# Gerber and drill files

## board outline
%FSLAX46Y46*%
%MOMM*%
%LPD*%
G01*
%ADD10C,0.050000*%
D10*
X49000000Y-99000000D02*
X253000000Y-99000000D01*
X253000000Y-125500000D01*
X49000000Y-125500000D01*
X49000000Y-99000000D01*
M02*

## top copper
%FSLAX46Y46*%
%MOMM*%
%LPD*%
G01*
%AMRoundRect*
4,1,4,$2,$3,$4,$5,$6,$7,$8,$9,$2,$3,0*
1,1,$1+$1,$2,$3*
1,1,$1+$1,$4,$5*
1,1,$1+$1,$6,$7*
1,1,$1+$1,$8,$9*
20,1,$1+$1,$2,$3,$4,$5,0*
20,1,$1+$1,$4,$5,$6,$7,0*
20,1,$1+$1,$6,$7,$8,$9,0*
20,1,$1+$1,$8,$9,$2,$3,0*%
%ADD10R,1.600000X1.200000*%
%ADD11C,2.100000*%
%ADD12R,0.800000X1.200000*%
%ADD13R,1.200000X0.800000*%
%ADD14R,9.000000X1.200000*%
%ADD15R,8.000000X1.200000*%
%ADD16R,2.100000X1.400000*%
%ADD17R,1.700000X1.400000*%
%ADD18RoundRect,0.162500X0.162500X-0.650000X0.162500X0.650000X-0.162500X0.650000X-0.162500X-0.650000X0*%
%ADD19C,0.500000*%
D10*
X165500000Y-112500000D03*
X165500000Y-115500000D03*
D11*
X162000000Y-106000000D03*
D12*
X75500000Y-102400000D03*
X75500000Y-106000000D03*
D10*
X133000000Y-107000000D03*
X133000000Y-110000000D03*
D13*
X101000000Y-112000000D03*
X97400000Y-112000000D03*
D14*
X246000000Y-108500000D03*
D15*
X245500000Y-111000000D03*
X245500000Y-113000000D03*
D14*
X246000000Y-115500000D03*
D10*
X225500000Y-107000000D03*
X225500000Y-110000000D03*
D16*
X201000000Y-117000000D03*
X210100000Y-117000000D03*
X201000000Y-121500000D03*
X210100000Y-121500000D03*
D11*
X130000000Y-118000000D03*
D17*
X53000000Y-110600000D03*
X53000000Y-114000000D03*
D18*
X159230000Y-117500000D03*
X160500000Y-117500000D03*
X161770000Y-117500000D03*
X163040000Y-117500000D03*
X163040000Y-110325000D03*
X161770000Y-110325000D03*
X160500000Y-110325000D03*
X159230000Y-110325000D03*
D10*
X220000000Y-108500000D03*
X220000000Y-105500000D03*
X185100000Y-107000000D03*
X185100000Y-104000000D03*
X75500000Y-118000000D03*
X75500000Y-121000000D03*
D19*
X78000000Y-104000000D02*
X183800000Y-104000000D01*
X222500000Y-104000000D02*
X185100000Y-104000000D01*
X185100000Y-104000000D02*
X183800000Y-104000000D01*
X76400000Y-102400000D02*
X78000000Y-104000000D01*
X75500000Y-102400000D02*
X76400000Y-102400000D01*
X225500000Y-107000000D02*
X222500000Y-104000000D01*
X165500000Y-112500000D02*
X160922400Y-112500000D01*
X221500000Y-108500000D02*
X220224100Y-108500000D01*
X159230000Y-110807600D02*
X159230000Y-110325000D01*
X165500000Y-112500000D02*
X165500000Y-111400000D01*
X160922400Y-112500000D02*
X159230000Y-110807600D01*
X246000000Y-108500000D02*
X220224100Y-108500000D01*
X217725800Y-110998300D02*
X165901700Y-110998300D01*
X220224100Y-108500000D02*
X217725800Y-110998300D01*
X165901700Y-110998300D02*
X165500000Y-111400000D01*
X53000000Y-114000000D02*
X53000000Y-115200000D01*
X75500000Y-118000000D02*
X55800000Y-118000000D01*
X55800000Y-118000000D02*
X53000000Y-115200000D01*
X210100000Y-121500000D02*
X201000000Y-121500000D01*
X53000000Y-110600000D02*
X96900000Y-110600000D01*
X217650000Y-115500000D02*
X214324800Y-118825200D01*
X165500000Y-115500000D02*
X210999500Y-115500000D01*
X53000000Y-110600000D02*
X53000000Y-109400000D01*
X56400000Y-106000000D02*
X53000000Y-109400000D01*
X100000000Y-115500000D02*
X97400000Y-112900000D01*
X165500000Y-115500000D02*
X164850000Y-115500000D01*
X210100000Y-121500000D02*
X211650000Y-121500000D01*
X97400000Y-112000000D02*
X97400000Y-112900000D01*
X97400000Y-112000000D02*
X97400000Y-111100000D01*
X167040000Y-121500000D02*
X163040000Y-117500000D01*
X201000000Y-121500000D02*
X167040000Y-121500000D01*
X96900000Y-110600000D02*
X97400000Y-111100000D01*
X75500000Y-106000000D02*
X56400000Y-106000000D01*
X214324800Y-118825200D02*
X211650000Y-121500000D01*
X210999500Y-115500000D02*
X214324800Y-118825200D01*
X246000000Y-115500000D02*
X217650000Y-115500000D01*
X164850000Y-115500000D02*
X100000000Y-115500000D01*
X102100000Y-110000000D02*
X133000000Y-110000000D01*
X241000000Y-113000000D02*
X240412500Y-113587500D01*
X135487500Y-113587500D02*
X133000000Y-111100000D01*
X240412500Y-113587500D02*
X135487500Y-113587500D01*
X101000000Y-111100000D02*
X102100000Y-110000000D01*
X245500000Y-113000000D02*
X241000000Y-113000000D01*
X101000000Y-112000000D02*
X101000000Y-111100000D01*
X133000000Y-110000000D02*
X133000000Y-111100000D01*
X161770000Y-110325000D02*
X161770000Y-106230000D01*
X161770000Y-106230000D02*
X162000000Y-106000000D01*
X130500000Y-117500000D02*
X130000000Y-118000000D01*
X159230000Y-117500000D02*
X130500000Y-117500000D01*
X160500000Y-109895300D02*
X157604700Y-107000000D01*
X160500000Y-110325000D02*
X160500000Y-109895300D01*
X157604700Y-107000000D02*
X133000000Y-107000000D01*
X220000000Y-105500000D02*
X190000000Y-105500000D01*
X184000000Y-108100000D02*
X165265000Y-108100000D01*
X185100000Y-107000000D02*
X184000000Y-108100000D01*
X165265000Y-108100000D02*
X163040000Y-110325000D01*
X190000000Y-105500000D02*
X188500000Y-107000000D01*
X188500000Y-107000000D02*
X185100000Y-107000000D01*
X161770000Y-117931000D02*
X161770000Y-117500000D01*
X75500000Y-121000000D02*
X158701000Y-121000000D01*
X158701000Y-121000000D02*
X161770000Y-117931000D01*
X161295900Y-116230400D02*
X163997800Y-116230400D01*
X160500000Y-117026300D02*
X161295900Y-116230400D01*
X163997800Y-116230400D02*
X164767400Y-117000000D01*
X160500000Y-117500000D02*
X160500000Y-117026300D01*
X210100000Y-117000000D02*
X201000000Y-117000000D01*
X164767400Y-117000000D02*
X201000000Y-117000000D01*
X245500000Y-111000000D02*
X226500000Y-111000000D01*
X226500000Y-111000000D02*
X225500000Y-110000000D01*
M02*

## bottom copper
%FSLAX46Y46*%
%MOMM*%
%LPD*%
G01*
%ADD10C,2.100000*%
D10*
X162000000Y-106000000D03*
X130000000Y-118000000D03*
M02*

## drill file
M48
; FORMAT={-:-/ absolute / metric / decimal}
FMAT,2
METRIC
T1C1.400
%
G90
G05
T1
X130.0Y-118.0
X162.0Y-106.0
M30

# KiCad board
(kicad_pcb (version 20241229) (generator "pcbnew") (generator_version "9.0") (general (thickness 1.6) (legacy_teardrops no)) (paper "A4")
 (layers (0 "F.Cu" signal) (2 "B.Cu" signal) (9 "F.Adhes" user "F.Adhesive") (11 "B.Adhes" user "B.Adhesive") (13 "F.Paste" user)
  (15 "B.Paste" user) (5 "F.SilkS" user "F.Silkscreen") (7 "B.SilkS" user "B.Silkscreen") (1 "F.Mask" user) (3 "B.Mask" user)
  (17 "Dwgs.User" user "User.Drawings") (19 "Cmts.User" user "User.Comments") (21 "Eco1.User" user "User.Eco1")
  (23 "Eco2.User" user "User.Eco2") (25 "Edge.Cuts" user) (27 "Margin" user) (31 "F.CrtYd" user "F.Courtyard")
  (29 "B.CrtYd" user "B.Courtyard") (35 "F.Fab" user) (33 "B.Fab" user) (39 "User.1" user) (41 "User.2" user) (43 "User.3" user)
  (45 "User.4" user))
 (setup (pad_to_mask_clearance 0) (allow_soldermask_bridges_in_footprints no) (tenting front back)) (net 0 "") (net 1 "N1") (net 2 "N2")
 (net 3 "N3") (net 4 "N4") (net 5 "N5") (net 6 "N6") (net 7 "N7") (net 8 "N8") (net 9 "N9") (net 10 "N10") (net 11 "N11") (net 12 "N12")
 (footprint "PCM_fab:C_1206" (layer "F.Cu") (at 165.5 114 -90)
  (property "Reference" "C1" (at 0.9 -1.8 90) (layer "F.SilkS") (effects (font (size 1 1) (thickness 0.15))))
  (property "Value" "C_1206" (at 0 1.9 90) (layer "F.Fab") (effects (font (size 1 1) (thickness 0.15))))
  (pad "1" smd rect (at -1.5 0 270) (size 1.2 1.6) (layers "F.Cu" "F.Mask" "F.Paste") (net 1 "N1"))
  (pad "2" smd rect (at 1.5 0 270) (size 1.2 1.6) (layers "F.Cu" "F.Mask" "F.Paste") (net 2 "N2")))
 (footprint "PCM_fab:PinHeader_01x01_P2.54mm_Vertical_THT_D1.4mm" (layer "F.Cu") (at 162 106)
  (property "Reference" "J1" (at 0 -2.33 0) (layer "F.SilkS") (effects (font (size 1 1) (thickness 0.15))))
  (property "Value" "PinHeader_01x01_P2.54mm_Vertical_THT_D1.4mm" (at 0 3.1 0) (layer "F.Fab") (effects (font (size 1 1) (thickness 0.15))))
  (pad "1" thru_hole circle (at 0 0) (size 2.1 2.1) (drill 1.4) (layers "*.Cu" "*.Mask") (remove_unused_layers no) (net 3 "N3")))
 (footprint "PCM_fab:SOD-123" (layer "F.Cu") (at 75.5 104.2 -90)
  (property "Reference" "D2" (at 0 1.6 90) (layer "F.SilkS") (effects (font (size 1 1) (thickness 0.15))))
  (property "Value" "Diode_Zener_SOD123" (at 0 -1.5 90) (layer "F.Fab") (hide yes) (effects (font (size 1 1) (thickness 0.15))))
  (pad "1" smd rect (at -1.8 0 270) (size 1.2 0.8) (layers "F.Cu" "F.Mask" "F.Paste") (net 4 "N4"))
  (pad "2" smd rect (at 1.8 0 270) (size 1.2 0.8) (layers "F.Cu" "F.Mask" "F.Paste") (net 2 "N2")))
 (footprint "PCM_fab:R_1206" (layer "F.Cu") (at 133 108.5 -90)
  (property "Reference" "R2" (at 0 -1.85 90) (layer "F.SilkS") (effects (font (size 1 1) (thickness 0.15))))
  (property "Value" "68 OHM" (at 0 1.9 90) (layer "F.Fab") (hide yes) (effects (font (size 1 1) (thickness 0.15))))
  (pad "1" smd rect (at -1.5 0 270) (size 1.2 1.6) (layers "F.Cu" "F.Mask" "F.Paste") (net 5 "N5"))
  (pad "2" smd rect (at 1.5 0 270) (size 1.2 1.6) (layers "F.Cu" "F.Mask" "F.Paste") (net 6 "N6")))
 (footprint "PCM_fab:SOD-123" (layer "F.Cu") (at 99.2 112 180)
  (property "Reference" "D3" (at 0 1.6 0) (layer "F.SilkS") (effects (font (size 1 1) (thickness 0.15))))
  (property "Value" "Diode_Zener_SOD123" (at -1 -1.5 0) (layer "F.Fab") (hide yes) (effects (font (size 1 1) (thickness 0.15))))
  (pad "1" smd rect (at -1.8 0 180) (size 1.2 0.8) (layers "F.Cu" "F.Mask" "F.Paste") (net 6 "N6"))
  (pad "2" smd rect (at 1.8 0 180) (size 1.2 0.8) (layers "F.Cu" "F.Mask" "F.Paste") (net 2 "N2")))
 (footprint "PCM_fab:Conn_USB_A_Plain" (layer "F.Cu") (at 246 112)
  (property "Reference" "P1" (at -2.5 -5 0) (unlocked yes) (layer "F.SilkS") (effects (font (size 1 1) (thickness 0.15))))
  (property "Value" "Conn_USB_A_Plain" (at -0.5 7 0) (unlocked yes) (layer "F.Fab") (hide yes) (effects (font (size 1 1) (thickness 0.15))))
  (pad "1" smd rect (at 0 -3.5) (size 9 1.2) (layers "F.Cu" "F.Mask" "F.Paste") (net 1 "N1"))
  (pad "2" smd rect (at -0.5 -1) (size 8 1.2) (layers "F.Cu" "F.Mask" "F.Paste") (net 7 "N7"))
  (pad "3" smd rect (at -0.5 1) (size 8 1.2) (layers "F.Cu" "F.Mask" "F.Paste") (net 6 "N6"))
  (pad "4" smd rect (at 0 3.5) (size 9 1.2) (layers "F.Cu" "F.Mask" "F.Paste") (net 2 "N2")))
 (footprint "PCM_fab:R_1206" (layer "F.Cu") (at 225.5 108.5 -90)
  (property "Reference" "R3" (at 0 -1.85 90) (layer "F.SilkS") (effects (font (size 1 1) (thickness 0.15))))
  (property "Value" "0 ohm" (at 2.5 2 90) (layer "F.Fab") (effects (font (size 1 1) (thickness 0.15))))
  (pad "1" smd rect (at -1.5 0 270) (size 1.2 1.6) (layers "F.Cu" "F.Mask" "F.Paste") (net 4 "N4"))
  (pad "2" smd rect (at 1.5 0 270) (size 1.2 1.6) (layers "F.Cu" "F.Mask" "F.Paste") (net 7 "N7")))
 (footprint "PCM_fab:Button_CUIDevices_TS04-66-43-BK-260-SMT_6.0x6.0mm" (layer "F.Cu") (at 205.55 119.25)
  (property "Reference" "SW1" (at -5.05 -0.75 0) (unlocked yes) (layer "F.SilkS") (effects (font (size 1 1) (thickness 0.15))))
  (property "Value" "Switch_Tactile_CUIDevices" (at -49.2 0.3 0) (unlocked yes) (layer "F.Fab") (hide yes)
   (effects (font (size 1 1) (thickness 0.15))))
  (pad "1" smd rect (at -4.55 -2.25) (size 2.1 1.4) (layers "F.Cu" "F.Mask" "F.Paste") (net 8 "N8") (thermal_bridge_angle 45))
  (pad "2" smd rect (at 4.55 -2.25) (size 2.1 1.4) (layers "F.Cu" "F.Mask" "F.Paste") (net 8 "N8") (thermal_bridge_angle 45))
  (pad "3" smd rect (at -4.55 2.25) (size 2.1 1.4) (layers "F.Cu" "F.Mask" "F.Paste") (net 2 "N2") (thermal_bridge_angle 45))
  (pad "4" smd rect (at 4.55 2.25) (size 2.1 1.4) (layers "F.Cu" "F.Mask" "F.Paste") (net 2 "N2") (thermal_bridge_angle 45)))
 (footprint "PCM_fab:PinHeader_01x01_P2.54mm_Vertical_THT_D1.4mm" (layer "F.Cu") (at 130 118)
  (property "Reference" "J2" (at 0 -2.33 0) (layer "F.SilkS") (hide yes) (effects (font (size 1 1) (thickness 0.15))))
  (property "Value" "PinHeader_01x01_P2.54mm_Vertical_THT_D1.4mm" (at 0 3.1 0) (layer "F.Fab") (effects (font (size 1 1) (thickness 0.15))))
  (pad "1" thru_hole circle (at 0 0) (size 2.1 2.1) (drill 1.4) (layers "*.Cu" "*.Mask") (remove_unused_layers no) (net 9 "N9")))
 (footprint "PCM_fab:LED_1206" (layer "F.Cu") (at 53 112.3 -90)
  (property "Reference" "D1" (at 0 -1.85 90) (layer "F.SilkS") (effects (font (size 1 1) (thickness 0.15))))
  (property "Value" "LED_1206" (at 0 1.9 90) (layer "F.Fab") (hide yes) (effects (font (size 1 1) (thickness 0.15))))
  (pad "1" smd rect (at -1.7 0 270) (size 1.4 1.7) (layers "F.Cu" "F.Mask" "F.Paste") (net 2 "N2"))
  (pad "2" smd rect (at 1.7 0 270) (size 1.4 1.7) (layers "F.Cu" "F.Mask" "F.Paste") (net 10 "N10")))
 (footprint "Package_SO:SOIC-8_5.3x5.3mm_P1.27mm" (layer "F.Cu") (at 161.135 113.9125 90)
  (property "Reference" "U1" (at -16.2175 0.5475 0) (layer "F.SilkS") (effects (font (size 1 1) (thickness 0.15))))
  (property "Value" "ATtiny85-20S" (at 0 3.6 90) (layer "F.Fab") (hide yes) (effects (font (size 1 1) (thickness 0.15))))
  (pad "1" smd roundrect (at -3.5875 -1.905 90) (size 1.625 0.65) (layers "F.Cu" "F.Mask" "F.Paste") (roundrect_rratio 0.25) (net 9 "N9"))
  (pad "2" smd roundrect (at -3.5875 -0.635 90) (size 1.625 0.65) (layers "F.Cu" "F.Mask" "F.Paste") (roundrect_rratio 0.25) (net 8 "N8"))
  (pad "3" smd roundrect (at -3.5875 0.635 90) (size 1.625 0.65) (layers "F.Cu" "F.Mask" "F.Paste") (roundrect_rratio 0.25) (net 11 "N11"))
  (pad "4" smd roundrect (at -3.5875 1.905 90) (size 1.625 0.65) (layers "F.Cu" "F.Mask" "F.Paste") (roundrect_rratio 0.25) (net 2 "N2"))
  (pad "5" smd roundrect (at 3.5875 1.905 90) (size 1.625 0.65) (layers "F.Cu" "F.Mask" "F.Paste") (roundrect_rratio 0.25) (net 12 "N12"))
  (pad "6" smd roundrect (at 3.5875 0.635 90) (size 1.625 0.65) (layers "F.Cu" "F.Mask" "F.Paste") (roundrect_rratio 0.25) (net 3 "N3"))
  (pad "7" smd roundrect (at 3.5875 -0.635 90) (size 1.625 0.65) (layers "F.Cu" "F.Mask" "F.Paste") (roundrect_rratio 0.25) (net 5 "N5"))
  (pad "8" smd roundrect (at 3.5875 -1.905 90) (size 1.625 0.65) (layers "F.Cu" "F.Mask" "F.Paste") (roundrect_rratio 0.25) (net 1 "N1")))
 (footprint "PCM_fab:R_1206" (layer "F.Cu") (at 220 107 90)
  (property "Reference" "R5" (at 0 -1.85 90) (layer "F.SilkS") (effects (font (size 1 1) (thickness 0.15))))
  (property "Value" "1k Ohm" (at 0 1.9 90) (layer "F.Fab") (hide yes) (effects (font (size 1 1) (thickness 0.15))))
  (pad "1" smd rect (at -1.5 0 90) (size 1.2 1.6) (layers "F.Cu" "F.Mask" "F.Paste") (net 1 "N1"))
  (pad "2" smd rect (at 1.5 0 90) (size 1.2 1.6) (layers "F.Cu" "F.Mask" "F.Paste") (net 12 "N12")))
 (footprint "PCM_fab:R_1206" (layer "F.Cu") (at 185.1 105.5 90)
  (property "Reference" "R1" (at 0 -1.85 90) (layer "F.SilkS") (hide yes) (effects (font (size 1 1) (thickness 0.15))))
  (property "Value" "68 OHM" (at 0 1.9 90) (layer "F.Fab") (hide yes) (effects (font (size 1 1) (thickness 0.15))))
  (pad "1" smd rect (at -1.5 0 90) (size 1.2 1.6) (layers "F.Cu" "F.Mask" "F.Paste") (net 12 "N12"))
  (pad "2" smd rect (at 1.5 0 90) (size 1.2 1.6) (layers "F.Cu" "F.Mask" "F.Paste") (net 4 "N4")))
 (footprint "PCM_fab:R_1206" (layer "F.Cu") (at 75.5 119.5 -90)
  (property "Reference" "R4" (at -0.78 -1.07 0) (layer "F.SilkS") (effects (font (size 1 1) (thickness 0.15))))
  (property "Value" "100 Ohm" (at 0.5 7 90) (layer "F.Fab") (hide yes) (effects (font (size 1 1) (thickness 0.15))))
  (pad "1" smd rect (at -1.5 0 270) (size 1.2 1.6) (layers "F.Cu" "F.Mask" "F.Paste") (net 10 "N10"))
  (pad "2" smd rect (at 1.5 0 270) (size 1.2 1.6) (layers "F.Cu" "F.Mask" "F.Paste") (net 11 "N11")))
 (gr_rect (start 49 99) (end 253 125.5) (stroke (width 0.05) (type default)) (fill no) (layer "Edge.Cuts"))
 (segment (start 78 104) (end 183.8 104) (width 0.5) (layer "F.Cu") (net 4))
 (segment (start 222.5 104) (end 185.1 104) (width 0.5) (layer "F.Cu") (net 4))
 (segment (start 185.1 104) (end 183.8 104) (width 0.5) (layer "F.Cu") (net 4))
 (segment (start 76.4 102.4) (end 78 104) (width 0.5) (layer "F.Cu") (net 4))
 (segment (start 75.5 102.4) (end 76.4 102.4) (width 0.5) (layer "F.Cu") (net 4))
 (segment (start 225.5 107) (end 222.5 104) (width 0.5) (layer "F.Cu") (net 4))
 (segment (start 165.5 112.5) (end 160.9224 112.5) (width 0.5) (layer "F.Cu") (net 1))
 (segment (start 221.5 108.5) (end 220.2241 108.5) (width 0.5) (layer "F.Cu") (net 1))
 (segment (start 159.23 110.8076) (end 159.23 110.325) (width 0.5) (layer "F.Cu") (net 1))
 (segment (start 165.5 112.5) (end 165.5 111.4) (width 0.5) (layer "F.Cu") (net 1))
 (segment (start 160.9224 112.5) (end 159.23 110.8076) (width 0.5) (layer "F.Cu") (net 1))
 (segment (start 246 108.5) (end 220.2241 108.5) (width 0.5) (layer "F.Cu") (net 1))
 (segment (start 217.7258 110.9983) (end 165.9017 110.9983) (width 0.5) (layer "F.Cu") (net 1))
 (segment (start 220.2241 108.5) (end 217.7258 110.9983) (width 0.5) (layer "F.Cu") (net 1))
 (segment (start 165.9017 110.9983) (end 165.5 111.4) (width 0.5) (layer "F.Cu") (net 1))
 (segment (start 53 114) (end 53 115.2) (width 0.5) (layer "F.Cu") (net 10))
 (segment (start 75.5 118) (end 55.8 118) (width 0.5) (layer "F.Cu") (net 10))
 (segment (start 55.8 118) (end 53 115.2) (width 0.5) (layer "F.Cu") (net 10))
 (segment (start 210.1 121.5) (end 201 121.5) (width 0.5) (layer "F.Cu") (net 2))
 (segment (start 53 110.6) (end 96.9 110.6) (width 0.5) (layer "F.Cu") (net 2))
 (segment (start 217.65 115.5) (end 214.3248 118.8252) (width 0.5) (layer "F.Cu") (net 2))
 (segment (start 165.5 115.5) (end 210.9995 115.5) (width 0.5) (layer "F.Cu") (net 2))
 (segment (start 53 110.6) (end 53 109.4) (width 0.5) (layer "F.Cu") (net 2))
 (segment (start 56.4 106) (end 53 109.4) (width 0.5) (layer "F.Cu") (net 2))
 (segment (start 100 115.5) (end 97.4 112.9) (width 0.5) (layer "F.Cu") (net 2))
 (segment (start 165.5 115.5) (end 164.85 115.5) (width 0.5) (layer "F.Cu") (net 2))
 (segment (start 210.1 121.5) (end 211.65 121.5) (width 0.5) (layer "F.Cu") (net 2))
 (segment (start 97.4 112) (end 97.4 112.9) (width 0.5) (layer "F.Cu") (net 2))
 (segment (start 97.4 112) (end 97.4 111.1) (width 0.5) (layer "F.Cu") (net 2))
 (segment (start 167.04 121.5) (end 163.04 117.5) (width 0.5) (layer "F.Cu") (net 2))
 (segment (start 201 121.5) (end 167.04 121.5) (width 0.5) (layer "F.Cu") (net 2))
 (segment (start 96.9 110.6) (end 97.4 111.1) (width 0.5) (layer "F.Cu") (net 2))
 (segment (start 75.5 106) (end 56.4 106) (width 0.5) (layer "F.Cu") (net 2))
 (segment (start 214.3248 118.8252) (end 211.65 121.5) (width 0.5) (layer "F.Cu") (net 2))
 (segment (start 210.9995 115.5) (end 214.3248 118.8252) (width 0.5) (layer "F.Cu") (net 2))
 (segment (start 246 115.5) (end 217.65 115.5) (width 0.5) (layer "F.Cu") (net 2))
 (segment (start 164.85 115.5) (end 100 115.5) (width 0.5) (layer "F.Cu") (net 2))
 (segment (start 102.1 110) (end 133 110) (width 0.5) (layer "F.Cu") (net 6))
 (segment (start 241 113) (end 240.4125 113.5875) (width 0.5) (layer "F.Cu") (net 6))
 (segment (start 135.4875 113.5875) (end 133 111.1) (width 0.5) (layer "F.Cu") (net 6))
 (segment (start 240.4125 113.5875) (end 135.4875 113.5875) (width 0.5) (layer "F.Cu") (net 6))
 (segment (start 101 111.1) (end 102.1 110) (width 0.5) (layer "F.Cu") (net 6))
 (segment (start 245.5 113) (end 241 113) (width 0.5) (layer "F.Cu") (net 6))
 (segment (start 101 112) (end 101 111.1) (width 0.5) (layer "F.Cu") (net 6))
 (segment (start 133 110) (end 133 111.1) (width 0.5) (layer "F.Cu") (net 6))
 (segment (start 161.77 110.325) (end 161.77 106.23) (width 0.5) (layer "F.Cu") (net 3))
 (segment (start 161.77 106.23) (end 162 106) (width 0.5) (layer "F.Cu") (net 3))
 (segment (start 130.5 117.5) (end 130 118) (width 0.5) (layer "F.Cu") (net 9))
 (segment (start 159.23 117.5) (end 130.5 117.5) (width 0.5) (layer "F.Cu") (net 9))
 (segment (start 160.5 109.8953) (end 157.6047 107) (width 0.5) (layer "F.Cu") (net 5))
 (segment (start 160.5 110.325) (end 160.5 109.8953) (width 0.5) (layer "F.Cu") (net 5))
 (segment (start 157.6047 107) (end 133 107) (width 0.5) (layer "F.Cu") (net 5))
 (segment (start 220 105.5) (end 190 105.5) (width 0.5) (layer "F.Cu") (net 12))
 (segment (start 184 108.1) (end 165.265 108.1) (width 0.5) (layer "F.Cu") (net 12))
 (segment (start 185.1 107) (end 184 108.1) (width 0.5) (layer "F.Cu") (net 12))
 (segment (start 165.265 108.1) (end 163.04 110.325) (width 0.5) (layer "F.Cu") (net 12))
 (segment (start 190 105.5) (end 188.5 107) (width 0.5) (layer "F.Cu") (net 12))
 (segment (start 188.5 107) (end 185.1 107) (width 0.5) (layer "F.Cu") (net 12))
 (segment (start 161.77 117.931) (end 161.77 117.5) (width 0.5) (layer "F.Cu") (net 11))
 (segment (start 75.5 121) (end 158.701 121) (width 0.5) (layer "F.Cu") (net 11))
 (segment (start 158.701 121) (end 161.77 117.931) (width 0.5) (layer "F.Cu") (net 11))
 (segment (start 161.2959 116.2304) (end 163.9978 116.2304) (width 0.5) (layer "F.Cu") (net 8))
 (segment (start 160.5 117.0263) (end 161.2959 116.2304) (width 0.5) (layer "F.Cu") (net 8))
 (segment (start 163.9978 116.2304) (end 164.7674 117) (width 0.5) (layer "F.Cu") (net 8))
 (segment (start 160.5 117.5) (end 160.5 117.0263) (width 0.5) (layer "F.Cu") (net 8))
 (segment (start 210.1 117) (end 201 117) (width 0.5) (layer "F.Cu") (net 8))
 (segment (start 164.7674 117) (end 201 117) (width 0.5) (layer "F.Cu") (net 8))
 (segment (start 245.5 111) (end 226.5 111) (width 0.5) (layer "F.Cu") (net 7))
 (segment (start 226.5 111) (end 225.5 110) (width 0.5) (layer "F.Cu") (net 7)))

